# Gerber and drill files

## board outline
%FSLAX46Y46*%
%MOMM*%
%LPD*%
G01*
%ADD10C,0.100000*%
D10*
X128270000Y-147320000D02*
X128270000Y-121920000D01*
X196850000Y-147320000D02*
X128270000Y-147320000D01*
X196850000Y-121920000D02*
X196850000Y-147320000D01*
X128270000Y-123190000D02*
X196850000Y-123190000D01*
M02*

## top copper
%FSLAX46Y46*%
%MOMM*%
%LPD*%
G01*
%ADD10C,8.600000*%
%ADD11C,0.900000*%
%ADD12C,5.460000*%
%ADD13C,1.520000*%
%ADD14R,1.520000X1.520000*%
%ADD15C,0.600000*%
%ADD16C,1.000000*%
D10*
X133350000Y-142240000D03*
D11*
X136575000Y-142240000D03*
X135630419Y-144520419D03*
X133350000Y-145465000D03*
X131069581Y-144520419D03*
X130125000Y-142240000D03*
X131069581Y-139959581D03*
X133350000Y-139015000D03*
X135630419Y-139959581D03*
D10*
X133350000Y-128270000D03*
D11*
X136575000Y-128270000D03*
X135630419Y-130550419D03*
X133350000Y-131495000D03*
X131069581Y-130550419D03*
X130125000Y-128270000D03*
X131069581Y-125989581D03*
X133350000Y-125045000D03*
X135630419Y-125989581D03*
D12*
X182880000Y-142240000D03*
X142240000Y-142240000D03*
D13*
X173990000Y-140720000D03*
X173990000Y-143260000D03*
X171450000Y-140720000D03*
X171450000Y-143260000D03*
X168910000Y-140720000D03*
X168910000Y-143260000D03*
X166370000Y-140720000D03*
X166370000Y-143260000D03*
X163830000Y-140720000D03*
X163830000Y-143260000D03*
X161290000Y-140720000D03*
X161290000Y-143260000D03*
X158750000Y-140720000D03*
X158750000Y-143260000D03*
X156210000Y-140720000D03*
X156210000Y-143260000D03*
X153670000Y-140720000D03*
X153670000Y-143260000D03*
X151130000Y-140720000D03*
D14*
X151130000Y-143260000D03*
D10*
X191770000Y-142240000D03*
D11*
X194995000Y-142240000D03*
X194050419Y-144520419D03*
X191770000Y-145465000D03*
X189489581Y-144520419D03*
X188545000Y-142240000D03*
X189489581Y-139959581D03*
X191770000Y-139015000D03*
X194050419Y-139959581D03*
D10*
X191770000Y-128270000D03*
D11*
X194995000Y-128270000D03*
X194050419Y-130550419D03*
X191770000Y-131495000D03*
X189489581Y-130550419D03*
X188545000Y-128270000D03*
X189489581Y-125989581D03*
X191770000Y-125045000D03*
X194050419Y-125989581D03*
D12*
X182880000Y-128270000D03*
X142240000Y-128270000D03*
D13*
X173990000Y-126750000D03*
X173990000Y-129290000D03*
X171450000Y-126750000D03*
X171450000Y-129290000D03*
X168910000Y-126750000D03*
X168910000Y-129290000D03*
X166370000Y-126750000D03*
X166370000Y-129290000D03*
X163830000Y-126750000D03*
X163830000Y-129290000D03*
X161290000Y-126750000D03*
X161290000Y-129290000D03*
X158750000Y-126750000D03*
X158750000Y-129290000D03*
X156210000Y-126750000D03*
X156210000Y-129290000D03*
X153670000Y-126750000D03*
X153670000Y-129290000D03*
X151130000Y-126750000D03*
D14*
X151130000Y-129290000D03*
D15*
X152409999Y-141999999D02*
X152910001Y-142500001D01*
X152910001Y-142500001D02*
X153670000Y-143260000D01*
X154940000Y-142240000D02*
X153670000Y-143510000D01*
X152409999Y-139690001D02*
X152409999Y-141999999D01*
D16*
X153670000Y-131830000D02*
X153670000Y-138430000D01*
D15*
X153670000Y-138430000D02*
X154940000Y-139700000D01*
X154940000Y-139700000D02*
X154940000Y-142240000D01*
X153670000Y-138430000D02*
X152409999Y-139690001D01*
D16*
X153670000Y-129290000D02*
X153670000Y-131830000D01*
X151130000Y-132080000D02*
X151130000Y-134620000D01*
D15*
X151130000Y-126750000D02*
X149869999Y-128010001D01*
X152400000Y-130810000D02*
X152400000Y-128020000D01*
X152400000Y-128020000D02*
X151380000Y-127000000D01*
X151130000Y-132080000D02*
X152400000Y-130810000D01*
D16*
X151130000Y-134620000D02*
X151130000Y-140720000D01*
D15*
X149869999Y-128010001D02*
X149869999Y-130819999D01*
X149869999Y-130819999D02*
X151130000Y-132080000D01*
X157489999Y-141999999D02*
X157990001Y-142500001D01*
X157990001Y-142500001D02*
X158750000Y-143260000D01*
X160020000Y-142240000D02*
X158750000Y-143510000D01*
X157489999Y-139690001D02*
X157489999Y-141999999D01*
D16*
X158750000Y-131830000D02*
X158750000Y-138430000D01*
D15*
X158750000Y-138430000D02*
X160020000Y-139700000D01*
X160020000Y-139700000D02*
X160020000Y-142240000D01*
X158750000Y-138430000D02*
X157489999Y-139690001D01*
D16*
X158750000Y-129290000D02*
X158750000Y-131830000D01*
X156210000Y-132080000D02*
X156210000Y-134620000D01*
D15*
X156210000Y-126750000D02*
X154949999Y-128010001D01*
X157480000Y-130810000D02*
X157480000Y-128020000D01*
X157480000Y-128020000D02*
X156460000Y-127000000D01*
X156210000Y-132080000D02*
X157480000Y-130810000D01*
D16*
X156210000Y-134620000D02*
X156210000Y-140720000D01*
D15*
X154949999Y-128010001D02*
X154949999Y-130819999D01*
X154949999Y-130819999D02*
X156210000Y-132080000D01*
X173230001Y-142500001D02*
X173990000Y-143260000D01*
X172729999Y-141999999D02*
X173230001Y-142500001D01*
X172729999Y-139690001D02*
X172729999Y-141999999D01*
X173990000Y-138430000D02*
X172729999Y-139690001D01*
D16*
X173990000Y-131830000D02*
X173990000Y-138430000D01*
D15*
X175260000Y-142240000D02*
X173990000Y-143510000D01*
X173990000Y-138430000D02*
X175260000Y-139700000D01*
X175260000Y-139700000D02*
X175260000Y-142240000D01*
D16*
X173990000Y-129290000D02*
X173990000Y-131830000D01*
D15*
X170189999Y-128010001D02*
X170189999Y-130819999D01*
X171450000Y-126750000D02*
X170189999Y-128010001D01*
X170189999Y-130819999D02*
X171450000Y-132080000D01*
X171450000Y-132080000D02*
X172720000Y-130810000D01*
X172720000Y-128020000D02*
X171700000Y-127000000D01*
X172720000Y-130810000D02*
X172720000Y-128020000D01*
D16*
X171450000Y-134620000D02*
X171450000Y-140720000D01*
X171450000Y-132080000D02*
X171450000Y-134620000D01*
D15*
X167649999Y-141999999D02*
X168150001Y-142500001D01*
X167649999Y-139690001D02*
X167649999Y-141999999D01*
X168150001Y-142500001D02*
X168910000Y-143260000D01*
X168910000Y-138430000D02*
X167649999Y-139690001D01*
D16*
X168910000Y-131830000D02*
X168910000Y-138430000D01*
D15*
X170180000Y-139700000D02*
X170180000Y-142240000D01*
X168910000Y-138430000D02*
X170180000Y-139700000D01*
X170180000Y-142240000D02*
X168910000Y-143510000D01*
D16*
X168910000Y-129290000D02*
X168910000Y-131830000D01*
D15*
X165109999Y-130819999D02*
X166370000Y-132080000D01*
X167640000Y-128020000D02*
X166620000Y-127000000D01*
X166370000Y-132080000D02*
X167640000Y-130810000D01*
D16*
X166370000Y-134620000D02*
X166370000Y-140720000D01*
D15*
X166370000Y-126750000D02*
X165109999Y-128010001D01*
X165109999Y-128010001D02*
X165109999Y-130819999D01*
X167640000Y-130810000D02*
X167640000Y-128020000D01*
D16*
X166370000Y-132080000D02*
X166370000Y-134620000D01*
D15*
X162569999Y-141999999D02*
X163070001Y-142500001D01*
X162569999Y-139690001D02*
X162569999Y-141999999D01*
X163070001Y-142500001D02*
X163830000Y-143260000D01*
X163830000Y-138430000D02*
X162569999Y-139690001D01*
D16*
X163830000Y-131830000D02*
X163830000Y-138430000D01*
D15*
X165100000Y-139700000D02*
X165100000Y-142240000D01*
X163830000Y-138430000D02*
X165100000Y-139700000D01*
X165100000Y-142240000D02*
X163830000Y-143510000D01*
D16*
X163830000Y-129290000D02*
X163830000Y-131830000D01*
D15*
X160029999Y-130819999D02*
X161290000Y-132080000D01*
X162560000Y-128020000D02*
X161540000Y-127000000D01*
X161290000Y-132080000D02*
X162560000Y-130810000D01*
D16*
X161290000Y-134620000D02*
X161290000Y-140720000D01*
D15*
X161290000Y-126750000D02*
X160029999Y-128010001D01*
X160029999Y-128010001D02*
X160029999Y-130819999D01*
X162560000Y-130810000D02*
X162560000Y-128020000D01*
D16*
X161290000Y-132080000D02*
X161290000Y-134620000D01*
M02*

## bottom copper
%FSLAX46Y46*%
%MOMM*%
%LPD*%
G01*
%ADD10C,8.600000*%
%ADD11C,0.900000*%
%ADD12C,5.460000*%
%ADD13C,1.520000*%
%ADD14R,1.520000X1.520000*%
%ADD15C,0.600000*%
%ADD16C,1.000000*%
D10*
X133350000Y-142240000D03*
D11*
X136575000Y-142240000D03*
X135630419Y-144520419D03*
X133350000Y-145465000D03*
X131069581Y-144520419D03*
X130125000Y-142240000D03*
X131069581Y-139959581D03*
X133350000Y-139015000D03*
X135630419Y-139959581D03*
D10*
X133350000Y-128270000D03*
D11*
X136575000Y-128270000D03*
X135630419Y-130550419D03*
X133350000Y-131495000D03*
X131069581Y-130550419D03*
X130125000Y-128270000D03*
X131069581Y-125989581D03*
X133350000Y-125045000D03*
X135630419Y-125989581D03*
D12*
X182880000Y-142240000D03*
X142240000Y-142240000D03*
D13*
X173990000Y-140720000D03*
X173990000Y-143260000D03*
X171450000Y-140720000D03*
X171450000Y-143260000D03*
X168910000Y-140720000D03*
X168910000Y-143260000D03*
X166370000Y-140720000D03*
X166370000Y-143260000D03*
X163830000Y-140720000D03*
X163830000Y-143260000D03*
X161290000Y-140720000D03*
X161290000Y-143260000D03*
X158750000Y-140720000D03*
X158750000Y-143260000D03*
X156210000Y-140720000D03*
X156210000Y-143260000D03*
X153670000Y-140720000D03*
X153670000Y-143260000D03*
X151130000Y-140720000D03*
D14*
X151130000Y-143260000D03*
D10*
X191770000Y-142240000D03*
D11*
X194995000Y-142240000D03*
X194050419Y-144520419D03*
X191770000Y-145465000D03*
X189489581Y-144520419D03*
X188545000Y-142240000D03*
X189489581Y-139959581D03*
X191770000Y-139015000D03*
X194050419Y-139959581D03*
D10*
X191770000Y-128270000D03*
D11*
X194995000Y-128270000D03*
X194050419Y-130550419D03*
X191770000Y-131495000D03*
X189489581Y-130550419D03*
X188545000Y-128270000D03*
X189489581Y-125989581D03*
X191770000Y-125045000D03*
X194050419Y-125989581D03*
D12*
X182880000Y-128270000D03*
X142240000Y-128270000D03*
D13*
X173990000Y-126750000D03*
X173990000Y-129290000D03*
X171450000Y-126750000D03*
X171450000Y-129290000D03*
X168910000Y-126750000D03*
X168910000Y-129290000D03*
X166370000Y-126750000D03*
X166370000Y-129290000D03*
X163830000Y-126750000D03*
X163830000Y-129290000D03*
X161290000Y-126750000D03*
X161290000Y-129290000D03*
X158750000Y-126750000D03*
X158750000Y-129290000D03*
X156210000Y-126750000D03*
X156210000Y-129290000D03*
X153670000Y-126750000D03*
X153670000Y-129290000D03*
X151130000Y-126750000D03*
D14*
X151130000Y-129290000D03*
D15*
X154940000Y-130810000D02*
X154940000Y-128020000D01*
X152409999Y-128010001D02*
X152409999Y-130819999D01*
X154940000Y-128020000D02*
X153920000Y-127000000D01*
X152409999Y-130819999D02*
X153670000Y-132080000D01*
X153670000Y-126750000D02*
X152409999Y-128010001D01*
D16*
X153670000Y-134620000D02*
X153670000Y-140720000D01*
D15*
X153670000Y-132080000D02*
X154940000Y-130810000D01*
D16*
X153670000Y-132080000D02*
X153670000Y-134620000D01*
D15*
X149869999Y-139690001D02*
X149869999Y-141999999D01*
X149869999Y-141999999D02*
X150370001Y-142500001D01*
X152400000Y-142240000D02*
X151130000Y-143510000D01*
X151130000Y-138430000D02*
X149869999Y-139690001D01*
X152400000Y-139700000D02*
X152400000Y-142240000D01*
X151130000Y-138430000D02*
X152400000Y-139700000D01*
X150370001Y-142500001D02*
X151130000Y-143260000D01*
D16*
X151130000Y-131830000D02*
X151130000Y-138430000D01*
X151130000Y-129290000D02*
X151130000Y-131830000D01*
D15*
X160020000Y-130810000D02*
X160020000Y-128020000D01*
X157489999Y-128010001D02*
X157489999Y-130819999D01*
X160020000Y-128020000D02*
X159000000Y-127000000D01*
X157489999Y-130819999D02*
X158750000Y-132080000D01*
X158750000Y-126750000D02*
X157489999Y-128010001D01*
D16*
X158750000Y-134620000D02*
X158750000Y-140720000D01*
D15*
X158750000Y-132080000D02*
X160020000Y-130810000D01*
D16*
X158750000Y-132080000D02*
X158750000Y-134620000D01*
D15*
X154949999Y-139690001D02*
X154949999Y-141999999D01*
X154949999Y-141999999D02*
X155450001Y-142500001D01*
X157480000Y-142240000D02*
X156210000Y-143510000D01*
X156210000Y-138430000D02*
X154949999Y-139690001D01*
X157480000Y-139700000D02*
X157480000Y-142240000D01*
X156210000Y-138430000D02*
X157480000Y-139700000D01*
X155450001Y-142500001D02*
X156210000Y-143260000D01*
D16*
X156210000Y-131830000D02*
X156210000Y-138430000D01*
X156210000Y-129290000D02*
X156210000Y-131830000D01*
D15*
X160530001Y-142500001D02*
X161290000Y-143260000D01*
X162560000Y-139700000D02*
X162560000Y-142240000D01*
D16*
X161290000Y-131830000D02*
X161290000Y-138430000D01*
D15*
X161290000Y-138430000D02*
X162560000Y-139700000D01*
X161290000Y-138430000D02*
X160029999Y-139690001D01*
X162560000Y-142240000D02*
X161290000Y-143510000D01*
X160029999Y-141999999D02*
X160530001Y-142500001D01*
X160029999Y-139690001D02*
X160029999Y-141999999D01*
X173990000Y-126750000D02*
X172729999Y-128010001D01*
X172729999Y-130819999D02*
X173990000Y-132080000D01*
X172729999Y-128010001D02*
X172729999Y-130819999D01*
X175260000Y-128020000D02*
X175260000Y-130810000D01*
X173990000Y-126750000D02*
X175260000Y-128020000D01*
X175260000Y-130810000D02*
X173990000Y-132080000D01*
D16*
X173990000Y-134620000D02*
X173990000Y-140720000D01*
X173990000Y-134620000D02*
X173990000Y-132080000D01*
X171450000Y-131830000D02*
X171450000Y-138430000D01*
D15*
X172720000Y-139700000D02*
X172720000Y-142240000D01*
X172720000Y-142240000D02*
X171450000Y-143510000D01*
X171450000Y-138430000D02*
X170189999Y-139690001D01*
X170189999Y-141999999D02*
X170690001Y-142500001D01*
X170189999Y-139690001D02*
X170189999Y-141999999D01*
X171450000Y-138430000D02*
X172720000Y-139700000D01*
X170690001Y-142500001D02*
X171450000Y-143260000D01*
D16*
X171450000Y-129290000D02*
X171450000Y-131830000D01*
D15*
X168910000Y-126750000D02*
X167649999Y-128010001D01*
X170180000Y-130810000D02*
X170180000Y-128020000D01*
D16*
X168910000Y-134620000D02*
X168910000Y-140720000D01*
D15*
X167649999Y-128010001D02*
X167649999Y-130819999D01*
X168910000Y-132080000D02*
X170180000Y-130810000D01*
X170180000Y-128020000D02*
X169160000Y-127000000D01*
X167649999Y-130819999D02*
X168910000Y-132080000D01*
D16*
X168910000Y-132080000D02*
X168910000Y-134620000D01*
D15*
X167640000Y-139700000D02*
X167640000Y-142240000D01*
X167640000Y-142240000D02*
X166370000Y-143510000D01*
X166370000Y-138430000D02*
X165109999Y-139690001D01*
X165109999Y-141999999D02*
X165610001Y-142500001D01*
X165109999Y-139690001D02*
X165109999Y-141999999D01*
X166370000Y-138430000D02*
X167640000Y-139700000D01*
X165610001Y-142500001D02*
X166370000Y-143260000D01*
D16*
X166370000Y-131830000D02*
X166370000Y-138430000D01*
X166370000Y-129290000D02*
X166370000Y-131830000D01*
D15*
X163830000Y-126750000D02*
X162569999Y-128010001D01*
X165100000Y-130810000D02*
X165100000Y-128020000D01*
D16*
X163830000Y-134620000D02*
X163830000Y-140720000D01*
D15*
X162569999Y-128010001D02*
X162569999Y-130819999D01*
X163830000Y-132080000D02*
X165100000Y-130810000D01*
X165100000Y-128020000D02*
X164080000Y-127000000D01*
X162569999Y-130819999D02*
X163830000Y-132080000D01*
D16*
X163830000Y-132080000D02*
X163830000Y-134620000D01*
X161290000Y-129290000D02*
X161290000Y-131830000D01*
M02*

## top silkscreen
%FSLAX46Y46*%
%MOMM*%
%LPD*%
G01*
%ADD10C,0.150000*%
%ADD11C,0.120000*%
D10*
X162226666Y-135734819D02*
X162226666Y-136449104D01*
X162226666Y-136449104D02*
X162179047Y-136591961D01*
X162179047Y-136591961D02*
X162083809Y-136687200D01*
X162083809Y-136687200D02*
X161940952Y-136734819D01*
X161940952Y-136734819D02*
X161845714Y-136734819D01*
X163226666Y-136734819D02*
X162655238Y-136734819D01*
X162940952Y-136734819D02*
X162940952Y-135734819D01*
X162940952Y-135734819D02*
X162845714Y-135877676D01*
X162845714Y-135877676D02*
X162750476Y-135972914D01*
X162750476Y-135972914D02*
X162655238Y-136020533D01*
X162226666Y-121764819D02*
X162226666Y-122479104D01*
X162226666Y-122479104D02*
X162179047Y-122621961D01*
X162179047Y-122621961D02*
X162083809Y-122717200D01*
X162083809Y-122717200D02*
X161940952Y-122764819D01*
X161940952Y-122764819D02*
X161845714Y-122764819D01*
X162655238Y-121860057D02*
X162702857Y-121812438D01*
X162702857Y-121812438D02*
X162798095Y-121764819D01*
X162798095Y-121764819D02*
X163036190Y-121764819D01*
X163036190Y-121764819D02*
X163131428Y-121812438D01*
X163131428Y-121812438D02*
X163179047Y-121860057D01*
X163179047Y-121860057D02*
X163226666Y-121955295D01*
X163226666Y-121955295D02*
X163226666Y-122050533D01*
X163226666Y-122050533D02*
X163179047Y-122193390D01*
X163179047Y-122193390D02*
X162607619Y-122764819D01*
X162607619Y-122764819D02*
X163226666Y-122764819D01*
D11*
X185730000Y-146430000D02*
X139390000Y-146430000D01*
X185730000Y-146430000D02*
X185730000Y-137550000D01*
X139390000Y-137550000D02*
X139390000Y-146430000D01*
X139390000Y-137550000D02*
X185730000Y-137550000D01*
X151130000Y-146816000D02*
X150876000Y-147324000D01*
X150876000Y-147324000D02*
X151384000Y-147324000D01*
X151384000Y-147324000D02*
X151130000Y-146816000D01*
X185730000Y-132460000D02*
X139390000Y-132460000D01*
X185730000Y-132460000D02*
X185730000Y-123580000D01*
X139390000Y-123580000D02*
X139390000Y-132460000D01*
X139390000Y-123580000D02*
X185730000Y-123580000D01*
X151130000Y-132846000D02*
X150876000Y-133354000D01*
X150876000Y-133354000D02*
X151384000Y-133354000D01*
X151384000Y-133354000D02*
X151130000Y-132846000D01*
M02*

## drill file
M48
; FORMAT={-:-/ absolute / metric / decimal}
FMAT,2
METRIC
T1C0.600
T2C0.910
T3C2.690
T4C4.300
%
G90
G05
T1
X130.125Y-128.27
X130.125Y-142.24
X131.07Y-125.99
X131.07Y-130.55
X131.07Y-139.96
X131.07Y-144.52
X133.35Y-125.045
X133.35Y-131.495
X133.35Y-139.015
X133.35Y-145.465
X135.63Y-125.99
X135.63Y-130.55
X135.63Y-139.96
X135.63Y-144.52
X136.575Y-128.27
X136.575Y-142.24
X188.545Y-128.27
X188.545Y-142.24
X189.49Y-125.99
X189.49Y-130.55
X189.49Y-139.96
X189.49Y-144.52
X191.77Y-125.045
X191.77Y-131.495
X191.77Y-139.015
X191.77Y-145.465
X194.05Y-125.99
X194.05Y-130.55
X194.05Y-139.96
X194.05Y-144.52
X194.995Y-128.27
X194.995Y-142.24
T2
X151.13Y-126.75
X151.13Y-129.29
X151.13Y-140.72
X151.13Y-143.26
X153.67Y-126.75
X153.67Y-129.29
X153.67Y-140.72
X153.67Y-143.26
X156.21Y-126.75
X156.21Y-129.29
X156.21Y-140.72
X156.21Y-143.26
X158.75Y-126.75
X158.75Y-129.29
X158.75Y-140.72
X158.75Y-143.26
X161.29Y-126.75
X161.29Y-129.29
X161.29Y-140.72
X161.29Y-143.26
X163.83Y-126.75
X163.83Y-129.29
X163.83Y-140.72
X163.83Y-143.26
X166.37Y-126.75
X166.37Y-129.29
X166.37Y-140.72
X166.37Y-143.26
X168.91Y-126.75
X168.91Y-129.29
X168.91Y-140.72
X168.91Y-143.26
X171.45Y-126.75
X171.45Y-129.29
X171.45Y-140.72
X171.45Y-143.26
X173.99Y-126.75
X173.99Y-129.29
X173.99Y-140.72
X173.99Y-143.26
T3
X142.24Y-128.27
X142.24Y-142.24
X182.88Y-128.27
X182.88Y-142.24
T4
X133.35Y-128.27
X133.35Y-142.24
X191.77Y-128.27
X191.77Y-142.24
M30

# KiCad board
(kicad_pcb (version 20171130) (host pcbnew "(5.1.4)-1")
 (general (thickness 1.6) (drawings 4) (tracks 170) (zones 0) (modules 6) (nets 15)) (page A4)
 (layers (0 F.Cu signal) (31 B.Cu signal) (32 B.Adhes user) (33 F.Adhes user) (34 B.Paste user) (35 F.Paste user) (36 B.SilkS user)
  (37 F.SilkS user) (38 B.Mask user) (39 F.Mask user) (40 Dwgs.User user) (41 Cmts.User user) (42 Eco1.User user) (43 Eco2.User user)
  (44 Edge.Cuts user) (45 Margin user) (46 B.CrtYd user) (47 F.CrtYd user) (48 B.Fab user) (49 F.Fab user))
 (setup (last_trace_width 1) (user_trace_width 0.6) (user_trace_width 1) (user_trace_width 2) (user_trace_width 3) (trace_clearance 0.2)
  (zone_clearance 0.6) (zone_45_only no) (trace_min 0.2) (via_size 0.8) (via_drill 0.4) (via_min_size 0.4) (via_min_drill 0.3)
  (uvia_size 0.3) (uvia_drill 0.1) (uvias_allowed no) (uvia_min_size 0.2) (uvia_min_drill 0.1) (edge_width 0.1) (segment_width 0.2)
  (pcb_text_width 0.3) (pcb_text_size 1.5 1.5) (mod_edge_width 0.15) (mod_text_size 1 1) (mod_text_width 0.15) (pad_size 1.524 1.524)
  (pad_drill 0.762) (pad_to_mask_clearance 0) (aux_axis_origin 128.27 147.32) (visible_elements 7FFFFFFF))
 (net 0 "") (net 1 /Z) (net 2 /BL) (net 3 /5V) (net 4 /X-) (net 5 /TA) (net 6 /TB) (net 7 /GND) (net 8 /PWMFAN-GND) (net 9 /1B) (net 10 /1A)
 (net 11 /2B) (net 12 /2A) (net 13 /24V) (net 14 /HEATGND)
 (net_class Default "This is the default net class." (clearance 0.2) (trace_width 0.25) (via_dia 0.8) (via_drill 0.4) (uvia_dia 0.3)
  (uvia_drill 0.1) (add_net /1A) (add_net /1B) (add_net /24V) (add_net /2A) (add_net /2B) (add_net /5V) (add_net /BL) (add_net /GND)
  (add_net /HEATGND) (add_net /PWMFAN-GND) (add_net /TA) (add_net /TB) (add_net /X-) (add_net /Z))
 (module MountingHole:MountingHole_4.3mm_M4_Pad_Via (layer F.Cu) (at 133.35 142.24)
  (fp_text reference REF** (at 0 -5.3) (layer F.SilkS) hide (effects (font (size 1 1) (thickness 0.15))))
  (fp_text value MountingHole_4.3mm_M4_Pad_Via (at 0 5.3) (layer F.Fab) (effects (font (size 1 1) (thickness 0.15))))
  (pad 1 thru_hole circle (at 0 0) (size 8.6 8.6) (drill 4.3) (layers *.Cu *.Mask))
  (pad 1 thru_hole circle (at 3.225 0) (size 0.9 0.9) (drill 0.6) (layers *.Cu *.Mask))
  (pad 1 thru_hole circle (at 2.280419 2.280419) (size 0.9 0.9) (drill 0.6) (layers *.Cu *.Mask))
  (pad 1 thru_hole circle (at 0 3.225) (size 0.9 0.9) (drill 0.6) (layers *.Cu *.Mask))
  (pad 1 thru_hole circle (at -2.280419 2.280419) (size 0.9 0.9) (drill 0.6) (layers *.Cu *.Mask))
  (pad 1 thru_hole circle (at -3.225 0) (size 0.9 0.9) (drill 0.6) (layers *.Cu *.Mask))
  (pad 1 thru_hole circle (at -2.280419 -2.280419) (size 0.9 0.9) (drill 0.6) (layers *.Cu *.Mask))
  (pad 1 thru_hole circle (at 0 -3.225) (size 0.9 0.9) (drill 0.6) (layers *.Cu *.Mask))
  (pad 1 thru_hole circle (at 2.280419 -2.280419) (size 0.9 0.9) (drill 0.6) (layers *.Cu *.Mask)))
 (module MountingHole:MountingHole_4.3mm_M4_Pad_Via (layer F.Cu) (at 133.35 128.27)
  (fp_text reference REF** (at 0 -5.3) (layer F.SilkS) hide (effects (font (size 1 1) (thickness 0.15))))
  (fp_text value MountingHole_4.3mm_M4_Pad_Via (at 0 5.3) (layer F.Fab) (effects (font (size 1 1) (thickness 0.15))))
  (pad 1 thru_hole circle (at 0 0) (size 8.6 8.6) (drill 4.3) (layers *.Cu *.Mask))
  (pad 1 thru_hole circle (at 3.225 0) (size 0.9 0.9) (drill 0.6) (layers *.Cu *.Mask))
  (pad 1 thru_hole circle (at 2.280419 2.280419) (size 0.9 0.9) (drill 0.6) (layers *.Cu *.Mask))
  (pad 1 thru_hole circle (at 0 3.225) (size 0.9 0.9) (drill 0.6) (layers *.Cu *.Mask))
  (pad 1 thru_hole circle (at -2.280419 2.280419) (size 0.9 0.9) (drill 0.6) (layers *.Cu *.Mask))
  (pad 1 thru_hole circle (at -3.225 0) (size 0.9 0.9) (drill 0.6) (layers *.Cu *.Mask))
  (pad 1 thru_hole circle (at -2.280419 -2.280419) (size 0.9 0.9) (drill 0.6) (layers *.Cu *.Mask))
  (pad 1 thru_hole circle (at 0 -3.225) (size 0.9 0.9) (drill 0.6) (layers *.Cu *.Mask))
  (pad 1 thru_hole circle (at 2.280419 -2.280419) (size 0.9 0.9) (drill 0.6) (layers *.Cu *.Mask)))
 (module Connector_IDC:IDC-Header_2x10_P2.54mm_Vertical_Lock (layer F.Cu) (at 151.13 143.26 90)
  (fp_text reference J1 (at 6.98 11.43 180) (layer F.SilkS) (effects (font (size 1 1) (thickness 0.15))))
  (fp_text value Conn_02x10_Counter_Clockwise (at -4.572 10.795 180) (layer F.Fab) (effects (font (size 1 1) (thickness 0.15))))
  (fp_line (start -3.17 34.6) (end -3.17 -11.74) (layer F.SilkS) (width 0.12))
  (fp_line (start -3.17 34.6) (end 5.71 34.6) (layer F.SilkS) (width 0.12))
  (fp_line (start 5.71 -11.74) (end -3.17 -11.74) (layer F.SilkS) (width 0.12))
  (fp_line (start 5.71 -11.74) (end 5.71 34.6) (layer F.SilkS) (width 0.12))
  (fp_line (start -3.556 0) (end -4.064 -0.254) (layer F.SilkS) (width 0.12))
  (fp_line (start -4.064 -0.254) (end -4.064 0.254) (layer F.SilkS) (width 0.12))
  (fp_line (start -4.064 0.254) (end -3.556 0) (layer F.SilkS) (width 0.12))
  (pad "" thru_hole circle (at 1.02 31.75) (size 5.46 5.46) (drill 2.69) (layers *.Cu *.Mask))
  (pad "" thru_hole circle (at 1.02 -8.89) (size 5.46 5.46) (drill 2.69) (layers *.Cu *.Mask))
  (pad 20 thru_hole circle (at 2.54 22.86) (size 1.52 1.52) (drill 0.91) (layers *.Cu *.Mask) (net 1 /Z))
  (pad 19 thru_hole circle (at 0 22.86) (size 1.52 1.52) (drill 0.91) (layers *.Cu *.Mask) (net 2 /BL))
  (pad 18 thru_hole circle (at 2.54 20.32) (size 1.52 1.52) (drill 0.91) (layers *.Cu *.Mask) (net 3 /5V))
  (pad 17 thru_hole circle (at 0 20.32) (size 1.52 1.52) (drill 0.91) (layers *.Cu *.Mask) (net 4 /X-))
  (pad 16 thru_hole circle (at 2.54 17.78) (size 1.52 1.52) (drill 0.91) (layers *.Cu *.Mask) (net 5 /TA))
  (pad 15 thru_hole circle (at 0 17.78) (size 1.52 1.52) (drill 0.91) (layers *.Cu *.Mask) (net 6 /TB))
  (pad 14 thru_hole circle (at 2.54 15.24) (size 1.52 1.52) (drill 0.91) (layers *.Cu *.Mask) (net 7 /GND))
  (pad 13 thru_hole circle (at 0 15.24) (size 1.52 1.52) (drill 0.91) (layers *.Cu *.Mask) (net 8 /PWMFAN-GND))
  (pad 12 thru_hole circle (at 2.54 12.7) (size 1.52 1.52) (drill 0.91) (layers *.Cu *.Mask) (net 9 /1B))
  (pad 11 thru_hole circle (at 0 12.7) (size 1.52 1.52) (drill 0.91) (layers *.Cu *.Mask) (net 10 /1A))
  (pad 10 thru_hole circle (at 2.54 10.16) (size 1.52 1.52) (drill 0.91) (layers *.Cu *.Mask) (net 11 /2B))
  (pad 9 thru_hole circle (at 0 10.16) (size 1.52 1.52) (drill 0.91) (layers *.Cu *.Mask) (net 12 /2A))
  (pad 8 thru_hole circle (at 2.54 7.62) (size 1.52 1.52) (drill 0.91) (layers *.Cu *.Mask) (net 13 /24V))
  (pad 7 thru_hole circle (at 0 7.62) (size 1.52 1.52) (drill 0.91) (layers *.Cu *.Mask) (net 13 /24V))
  (pad 6 thru_hole circle (at 2.54 5.08) (size 1.52 1.52) (drill 0.91) (layers *.Cu *.Mask) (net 13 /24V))
  (pad 5 thru_hole circle (at 0 5.08) (size 1.52 1.52) (drill 0.91) (layers *.Cu *.Mask) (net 13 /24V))
  (pad 4 thru_hole circle (at 2.54 2.54) (size 1.52 1.52) (drill 0.91) (layers *.Cu *.Mask) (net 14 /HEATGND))
  (pad 3 thru_hole circle (at 0 2.54) (size 1.52 1.52) (drill 0.91) (layers *.Cu *.Mask) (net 14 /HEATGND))
  (pad 2 thru_hole circle (at 2.54 0) (size 1.52 1.52) (drill 0.91) (layers *.Cu *.Mask) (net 14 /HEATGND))
  (pad 1 thru_hole rect (at 0 0) (size 1.52 1.52) (drill 0.91) (layers *.Cu *.Mask) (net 14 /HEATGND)))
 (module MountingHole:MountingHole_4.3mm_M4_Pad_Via (layer F.Cu) (at 191.77 142.24)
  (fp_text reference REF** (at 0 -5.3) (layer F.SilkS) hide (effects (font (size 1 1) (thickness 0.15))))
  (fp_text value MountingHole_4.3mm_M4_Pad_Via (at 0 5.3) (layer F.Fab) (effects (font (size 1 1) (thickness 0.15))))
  (pad 1 thru_hole circle (at 0 0) (size 8.6 8.6) (drill 4.3) (layers *.Cu *.Mask))
  (pad 1 thru_hole circle (at 3.225 0) (size 0.9 0.9) (drill 0.6) (layers *.Cu *.Mask))
  (pad 1 thru_hole circle (at 2.280419 2.280419) (size 0.9 0.9) (drill 0.6) (layers *.Cu *.Mask))
  (pad 1 thru_hole circle (at 0 3.225) (size 0.9 0.9) (drill 0.6) (layers *.Cu *.Mask))
  (pad 1 thru_hole circle (at -2.280419 2.280419) (size 0.9 0.9) (drill 0.6) (layers *.Cu *.Mask))
  (pad 1 thru_hole circle (at -3.225 0) (size 0.9 0.9) (drill 0.6) (layers *.Cu *.Mask))
  (pad 1 thru_hole circle (at -2.280419 -2.280419) (size 0.9 0.9) (drill 0.6) (layers *.Cu *.Mask))
  (pad 1 thru_hole circle (at 0 -3.225) (size 0.9 0.9) (drill 0.6) (layers *.Cu *.Mask))
  (pad 1 thru_hole circle (at 2.280419 -2.280419) (size 0.9 0.9) (drill 0.6) (layers *.Cu *.Mask)))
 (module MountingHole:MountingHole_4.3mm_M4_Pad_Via (layer F.Cu) (at 191.77 128.27)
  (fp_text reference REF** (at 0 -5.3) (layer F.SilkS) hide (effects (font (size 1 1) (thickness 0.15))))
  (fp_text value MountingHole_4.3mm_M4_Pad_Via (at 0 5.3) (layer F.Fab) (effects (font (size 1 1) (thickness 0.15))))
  (pad 1 thru_hole circle (at 0 0) (size 8.6 8.6) (drill 4.3) (layers *.Cu *.Mask))
  (pad 1 thru_hole circle (at 3.225 0) (size 0.9 0.9) (drill 0.6) (layers *.Cu *.Mask))
  (pad 1 thru_hole circle (at 2.280419 2.280419) (size 0.9 0.9) (drill 0.6) (layers *.Cu *.Mask))
  (pad 1 thru_hole circle (at 0 3.225) (size 0.9 0.9) (drill 0.6) (layers *.Cu *.Mask))
  (pad 1 thru_hole circle (at -2.280419 2.280419) (size 0.9 0.9) (drill 0.6) (layers *.Cu *.Mask))
  (pad 1 thru_hole circle (at -3.225 0) (size 0.9 0.9) (drill 0.6) (layers *.Cu *.Mask))
  (pad 1 thru_hole circle (at -2.280419 -2.280419) (size 0.9 0.9) (drill 0.6) (layers *.Cu *.Mask))
  (pad 1 thru_hole circle (at 0 -3.225) (size 0.9 0.9) (drill 0.6) (layers *.Cu *.Mask))
  (pad 1 thru_hole circle (at 2.280419 -2.280419) (size 0.9 0.9) (drill 0.6) (layers *.Cu *.Mask)))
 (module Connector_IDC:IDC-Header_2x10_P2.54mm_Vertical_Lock (layer F.Cu) (at 151.13 129.29 90)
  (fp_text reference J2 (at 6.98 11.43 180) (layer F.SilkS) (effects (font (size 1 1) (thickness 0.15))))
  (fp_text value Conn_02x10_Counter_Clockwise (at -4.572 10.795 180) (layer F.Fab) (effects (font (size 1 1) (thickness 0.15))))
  (fp_line (start -3.17 34.6) (end -3.17 -11.74) (layer F.SilkS) (width 0.12))
  (fp_line (start -3.17 34.6) (end 5.71 34.6) (layer F.SilkS) (width 0.12))
  (fp_line (start 5.71 -11.74) (end -3.17 -11.74) (layer F.SilkS) (width 0.12))
  (fp_line (start 5.71 -11.74) (end 5.71 34.6) (layer F.SilkS) (width 0.12))
  (fp_line (start -3.556 0) (end -4.064 -0.254) (layer F.SilkS) (width 0.12))
  (fp_line (start -4.064 -0.254) (end -4.064 0.254) (layer F.SilkS) (width 0.12))
  (fp_line (start -4.064 0.254) (end -3.556 0) (layer F.SilkS) (width 0.12))
  (pad "" thru_hole circle (at 1.02 31.75) (size 5.46 5.46) (drill 2.69) (layers *.Cu *.Mask))
  (pad "" thru_hole circle (at 1.02 -8.89) (size 5.46 5.46) (drill 2.69) (layers *.Cu *.Mask))
  (pad 20 thru_hole circle (at 2.54 22.86) (size 1.52 1.52) (drill 0.91) (layers *.Cu *.Mask) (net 1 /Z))
  (pad 19 thru_hole circle (at 0 22.86) (size 1.52 1.52) (drill 0.91) (layers *.Cu *.Mask) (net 2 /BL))
  (pad 18 thru_hole circle (at 2.54 20.32) (size 1.52 1.52) (drill 0.91) (layers *.Cu *.Mask) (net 3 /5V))
  (pad 17 thru_hole circle (at 0 20.32) (size 1.52 1.52) (drill 0.91) (layers *.Cu *.Mask) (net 4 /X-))
  (pad 16 thru_hole circle (at 2.54 17.78) (size 1.52 1.52) (drill 0.91) (layers *.Cu *.Mask) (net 5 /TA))
  (pad 15 thru_hole circle (at 0 17.78) (size 1.52 1.52) (drill 0.91) (layers *.Cu *.Mask) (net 6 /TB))
  (pad 14 thru_hole circle (at 2.54 15.24) (size 1.52 1.52) (drill 0.91) (layers *.Cu *.Mask) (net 7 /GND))
  (pad 13 thru_hole circle (at 0 15.24) (size 1.52 1.52) (drill 0.91) (layers *.Cu *.Mask) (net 8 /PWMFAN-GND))
  (pad 12 thru_hole circle (at 2.54 12.7) (size 1.52 1.52) (drill 0.91) (layers *.Cu *.Mask) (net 9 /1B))
  (pad 11 thru_hole circle (at 0 12.7) (size 1.52 1.52) (drill 0.91) (layers *.Cu *.Mask) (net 10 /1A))
  (pad 10 thru_hole circle (at 2.54 10.16) (size 1.52 1.52) (drill 0.91) (layers *.Cu *.Mask) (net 11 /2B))
  (pad 9 thru_hole circle (at 0 10.16) (size 1.52 1.52) (drill 0.91) (layers *.Cu *.Mask) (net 12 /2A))
  (pad 8 thru_hole circle (at 2.54 7.62) (size 1.52 1.52) (drill 0.91) (layers *.Cu *.Mask) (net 13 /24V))
  (pad 7 thru_hole circle (at 0 7.62) (size 1.52 1.52) (drill 0.91) (layers *.Cu *.Mask) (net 13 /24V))
  (pad 6 thru_hole circle (at 2.54 5.08) (size 1.52 1.52) (drill 0.91) (layers *.Cu *.Mask) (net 13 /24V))
  (pad 5 thru_hole circle (at 0 5.08) (size 1.52 1.52) (drill 0.91) (layers *.Cu *.Mask) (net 13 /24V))
  (pad 4 thru_hole circle (at 2.54 2.54) (size 1.52 1.52) (drill 0.91) (layers *.Cu *.Mask) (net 14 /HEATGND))
  (pad 3 thru_hole circle (at 0 2.54) (size 1.52 1.52) (drill 0.91) (layers *.Cu *.Mask) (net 14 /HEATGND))
  (pad 2 thru_hole circle (at 2.54 0) (size 1.52 1.52) (drill 0.91) (layers *.Cu *.Mask) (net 14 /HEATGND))
  (pad 1 thru_hole rect (at 0 0) (size 1.52 1.52) (drill 0.91) (layers *.Cu *.Mask) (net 14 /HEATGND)))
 (gr_line (start 128.27 147.32) (end 128.27 121.92) (layer Edge.Cuts) (width 0.1))
 (gr_line (start 196.85 147.32) (end 128.27 147.32) (layer Edge.Cuts) (width 0.1))
 (gr_line (start 196.85 121.92) (end 196.85 147.32) (layer Edge.Cuts) (width 0.1))
 (gr_line (start 128.27 123.19) (end 196.85 123.19) (layer Edge.Cuts) (width 0.1))
 (segment (start 154.94 130.81) (end 154.94 128.02) (width 0.6) (layer B.Cu) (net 14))
 (segment (start 152.409999 128.010001) (end 152.409999 130.819999) (width 0.6) (layer B.Cu) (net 14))
 (segment (start 154.94 128.02) (end 153.92 127) (width 0.6) (layer B.Cu) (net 14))
 (segment (start 152.409999 130.819999) (end 153.67 132.08) (width 0.6) (layer B.Cu) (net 14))
 (segment (start 153.67 126.75) (end 152.409999 128.010001) (width 0.6) (layer B.Cu) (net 14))
 (segment (start 153.67 134.62) (end 153.67 140.72) (width 1) (layer B.Cu) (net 14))
 (segment (start 153.67 132.08) (end 154.94 130.81) (width 0.6) (layer B.Cu) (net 14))
 (segment (start 153.67 132.08) (end 153.67 134.62) (width 1) (layer B.Cu) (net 14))
 (segment (start 149.869999 139.690001) (end 149.869999 141.999999) (width 0.6) (layer B.Cu) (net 14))
 (segment (start 149.869999 141.999999) (end 150.370001 142.500001) (width 0.6) (layer B.Cu) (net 14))
 (segment (start 152.4 142.24) (end 151.13 143.51) (width 0.6) (layer B.Cu) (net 14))
 (segment (start 151.13 138.43) (end 149.869999 139.690001) (width 0.6) (layer B.Cu) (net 14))
 (segment (start 152.4 139.7) (end 152.4 142.24) (width 0.6) (layer B.Cu) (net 14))
 (segment (start 151.13 138.43) (end 152.4 139.7) (width 0.6) (layer B.Cu) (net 14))
 (segment (start 150.370001 142.500001) (end 151.13 143.26) (width 0.6) (layer B.Cu) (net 14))
 (segment (start 151.13 131.83) (end 151.13 138.43) (width 1) (layer B.Cu) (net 14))
 (segment (start 151.13 129.29) (end 151.13 131.83) (width 1) (layer B.Cu) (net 14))
 (segment (start 160.02 130.81) (end 160.02 128.02) (width 0.6) (layer B.Cu) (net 13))
 (segment (start 157.489999 128.010001) (end 157.489999 130.819999) (width 0.6) (layer B.Cu) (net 13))
 (segment (start 160.02 128.02) (end 159 127) (width 0.6) (layer B.Cu) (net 13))
 (segment (start 157.489999 130.819999) (end 158.75 132.08) (width 0.6) (layer B.Cu) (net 13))
 (segment (start 158.75 126.75) (end 157.489999 128.010001) (width 0.6) (layer B.Cu) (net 13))
 (segment (start 158.75 134.62) (end 158.75 140.72) (width 1) (layer B.Cu) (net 13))
 (segment (start 158.75 132.08) (end 160.02 130.81) (width 0.6) (layer B.Cu) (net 13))
 (segment (start 158.75 132.08) (end 158.75 134.62) (width 1) (layer B.Cu) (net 13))
 (segment (start 154.949999 139.690001) (end 154.949999 141.999999) (width 0.6) (layer B.Cu) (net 13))
 (segment (start 154.949999 141.999999) (end 155.450001 142.500001) (width 0.6) (layer B.Cu) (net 13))
 (segment (start 157.48 142.24) (end 156.21 143.51) (width 0.6) (layer B.Cu) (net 13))
 (segment (start 156.21 138.43) (end 154.949999 139.690001) (width 0.6) (layer B.Cu) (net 13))
 (segment (start 157.48 139.7) (end 157.48 142.24) (width 0.6) (layer B.Cu) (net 13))
 (segment (start 156.21 138.43) (end 157.48 139.7) (width 0.6) (layer B.Cu) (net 13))
 (segment (start 155.450001 142.500001) (end 156.21 143.26) (width 0.6) (layer B.Cu) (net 13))
 (segment (start 156.21 131.83) (end 156.21 138.43) (width 1) (layer B.Cu) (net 13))
 (segment (start 156.21 129.29) (end 156.21 131.83) (width 1) (layer B.Cu) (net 13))
 (segment (start 152.409999 141.999999) (end 152.910001 142.500001) (width 0.6) (layer F.Cu) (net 14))
 (segment (start 152.910001 142.500001) (end 153.67 143.26) (width 0.6) (layer F.Cu) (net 14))
 (segment (start 154.94 142.24) (end 153.67 143.51) (width 0.6) (layer F.Cu) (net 14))
 (segment (start 152.409999 139.690001) (end 152.409999 141.999999) (width 0.6) (layer F.Cu) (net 14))
 (segment (start 153.67 131.83) (end 153.67 138.43) (width 1) (layer F.Cu) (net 14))
 (segment (start 153.67 138.43) (end 154.94 139.7) (width 0.6) (layer F.Cu) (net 14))
 (segment (start 154.94 139.7) (end 154.94 142.24) (width 0.6) (layer F.Cu) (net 14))
 (segment (start 153.67 138.43) (end 152.409999 139.690001) (width 0.6) (layer F.Cu) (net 14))
 (segment (start 153.67 129.29) (end 153.67 131.83) (width 1) (layer F.Cu) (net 14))
 (segment (start 151.13 132.08) (end 151.13 134.62) (width 1) (layer F.Cu) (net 14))
 (segment (start 151.13 126.75) (end 149.869999 128.010001) (width 0.6) (layer F.Cu) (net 14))
 (segment (start 152.4 130.81) (end 152.4 128.02) (width 0.6) (layer F.Cu) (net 14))
 (segment (start 152.4 128.02) (end 151.38 127) (width 0.6) (layer F.Cu) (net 14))
 (segment (start 151.13 132.08) (end 152.4 130.81) (width 0.6) (layer F.Cu) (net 14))
 (segment (start 151.13 134.62) (end 151.13 140.72) (width 1) (layer F.Cu) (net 14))
 (segment (start 149.869999 128.010001) (end 149.869999 130.819999) (width 0.6) (layer F.Cu) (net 14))
 (segment (start 149.869999 130.819999) (end 151.13 132.08) (width 0.6) (layer F.Cu) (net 14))
 (segment (start 157.489999 141.999999) (end 157.990001 142.500001) (width 0.6) (layer F.Cu) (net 13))
 (segment (start 157.990001 142.500001) (end 158.75 143.26) (width 0.6) (layer F.Cu) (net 13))
 (segment (start 160.02 142.24) (end 158.75 143.51) (width 0.6) (layer F.Cu) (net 13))
 (segment (start 157.489999 139.690001) (end 157.489999 141.999999) (width 0.6) (layer F.Cu) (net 13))
 (segment (start 158.75 131.83) (end 158.75 138.43) (width 1) (layer F.Cu) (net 13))
 (segment (start 158.75 138.43) (end 160.02 139.7) (width 0.6) (layer F.Cu) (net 13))
 (segment (start 160.02 139.7) (end 160.02 142.24) (width 0.6) (layer F.Cu) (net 13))
 (segment (start 158.75 138.43) (end 157.489999 139.690001) (width 0.6) (layer F.Cu) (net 13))
 (segment (start 158.75 129.29) (end 158.75 131.83) (width 1) (layer F.Cu) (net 13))
 (segment (start 156.21 132.08) (end 156.21 134.62) (width 1) (layer F.Cu) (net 13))
 (segment (start 156.21 126.75) (end 154.949999 128.010001) (width 0.6) (layer F.Cu) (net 13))
 (segment (start 157.48 130.81) (end 157.48 128.02) (width 0.6) (layer F.Cu) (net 13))
 (segment (start 157.48 128.02) (end 156.46 127) (width 0.6) (layer F.Cu) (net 13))
 (segment (start 156.21 132.08) (end 157.48 130.81) (width 0.6) (layer F.Cu) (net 13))
 (segment (start 156.21 134.62) (end 156.21 140.72) (width 1) (layer F.Cu) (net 13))
 (segment (start 154.949999 128.010001) (end 154.949999 130.819999) (width 0.6) (layer F.Cu) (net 13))
 (segment (start 154.949999 130.819999) (end 156.21 132.08) (width 0.6) (layer F.Cu) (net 13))
 (segment (start 160.530001 142.500001) (end 161.29 143.26) (width 0.6) (layer B.Cu) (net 12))
 (segment (start 162.56 139.7) (end 162.56 142.24) (width 0.6) (layer B.Cu) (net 12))
 (segment (start 161.29 131.83) (end 161.29 138.43) (width 1) (layer B.Cu) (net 12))
 (segment (start 161.29 138.43) (end 162.56 139.7) (width 0.6) (layer B.Cu) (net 12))
 (segment (start 161.29 138.43) (end 160.029999 139.690001) (width 0.6) (layer B.Cu) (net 12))
 (segment (start 162.56 142.24) (end 161.29 143.51) (width 0.6) (layer B.Cu) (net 12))
 (segment (start 160.029999 141.999999) (end 160.530001 142.500001) (width 0.6) (layer B.Cu) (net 12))
 (segment (start 160.029999 139.690001) (end 160.029999 141.999999) (width 0.6) (layer B.Cu) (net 12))
 (segment (start 173.99 126.75) (end 172.729999 128.010001) (width 0.6) (layer B.Cu) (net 1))
 (segment (start 172.729999 130.819999) (end 173.99 132.08) (width 0.6) (layer B.Cu) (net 1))
 (segment (start 172.729999 128.010001) (end 172.729999 130.819999) (width 0.6) (layer B.Cu) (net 1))
 (segment (start 175.26 128.02) (end 175.26 130.81) (width 0.6) (layer B.Cu) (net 1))
 (segment (start 173.99 126.75) (end 175.26 128.02) (width 0.6) (layer B.Cu) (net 1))
 (segment (start 175.26 130.81) (end 173.99 132.08) (width 0.6) (layer B.Cu) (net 1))
 (segment (start 173.99 134.62) (end 173.99 140.72) (width 1) (layer B.Cu) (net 1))
 (segment (start 173.99 134.62) (end 173.99 132.08) (width 1) (layer B.Cu) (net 1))
 (segment (start 173.230001 142.500001) (end 173.99 143.26) (width 0.6) (layer F.Cu) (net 2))
 (segment (start 172.729999 141.999999) (end 173.230001 142.500001) (width 0.6) (layer F.Cu) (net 2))
 (segment (start 172.729999 139.690001) (end 172.729999 141.999999) (width 0.6) (layer F.Cu) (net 2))
 (segment (start 173.99 138.43) (end 172.729999 139.690001) (width 0.6) (layer F.Cu) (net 2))
 (segment (start 173.99 131.83) (end 173.99 138.43) (width 1) (layer F.Cu) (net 2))
 (segment (start 175.26 142.24) (end 173.99 143.51) (width 0.6) (layer F.Cu) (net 2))
 (segment (start 173.99 138.43) (end 175.26 139.7) (width 0.6) (layer F.Cu) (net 2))
 (segment (start 175.26 139.7) (end 175.26 142.24) (width 0.6) (layer F.Cu) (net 2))
 (segment (start 173.99 129.29) (end 173.99 131.83) (width 1) (layer F.Cu) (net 2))
 (segment (start 170.189999 128.010001) (end 170.189999 130.819999) (width 0.6) (layer F.Cu) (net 3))
 (segment (start 171.45 126.75) (end 170.189999 128.010001) (width 0.6) (layer F.Cu) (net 3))
 (segment (start 170.189999 130.819999) (end 171.45 132.08) (width 0.6) (layer F.Cu) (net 3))
 (segment (start 171.45 132.08) (end 172.72 130.81) (width 0.6) (layer F.Cu) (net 3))
 (segment (start 172.72 128.02) (end 171.7 127) (width 0.6) (layer F.Cu) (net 3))
 (segment (start 172.72 130.81) (end 172.72 128.02) (width 0.6) (layer F.Cu) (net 3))
 (segment (start 171.45 134.62) (end 171.45 140.72) (width 1) (layer F.Cu) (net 3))
 (segment (start 171.45 132.08) (end 171.45 134.62) (width 1) (layer F.Cu) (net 3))
 (segment (start 171.45 131.83) (end 171.45 138.43) (width 1) (layer B.Cu) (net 4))
 (segment (start 172.72 139.7) (end 172.72 142.24) (width 0.6) (layer B.Cu) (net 4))
 (segment (start 172.72 142.24) (end 171.45 143.51) (width 0.6) (layer B.Cu) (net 4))
 (segment (start 171.45 138.43) (end 170.189999 139.690001) (width 0.6) (layer B.Cu) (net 4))
 (segment (start 170.189999 141.999999) (end 170.690001 142.500001) (width 0.6) (layer B.Cu) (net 4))
 (segment (start 170.189999 139.690001) (end 170.189999 141.999999) (width 0.6) (layer B.Cu) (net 4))
 (segment (start 171.45 138.43) (end 172.72 139.7) (width 0.6) (layer B.Cu) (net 4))
 (segment (start 170.690001 142.500001) (end 171.45 143.26) (width 0.6) (layer B.Cu) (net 4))
 (segment (start 171.45 129.29) (end 171.45 131.83) (width 1) (layer B.Cu) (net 4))
 (segment (start 168.91 126.75) (end 167.649999 128.010001) (width 0.6) (layer B.Cu) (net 5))
 (segment (start 170.18 130.81) (end 170.18 128.02) (width 0.6) (layer B.Cu) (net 5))
 (segment (start 168.91 134.62) (end 168.91 140.72) (width 1) (layer B.Cu) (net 5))
 (segment (start 167.649999 128.010001) (end 167.649999 130.819999) (width 0.6) (layer B.Cu) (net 5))
 (segment (start 168.91 132.08) (end 170.18 130.81) (width 0.6) (layer B.Cu) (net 5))
 (segment (start 170.18 128.02) (end 169.16 127) (width 0.6) (layer B.Cu) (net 5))
 (segment (start 167.649999 130.819999) (end 168.91 132.08) (width 0.6) (layer B.Cu) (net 5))
 (segment (start 168.91 132.08) (end 168.91 134.62) (width 1) (layer B.Cu) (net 5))
 (segment (start 167.649999 141.999999) (end 168.150001 142.500001) (width 0.6) (layer F.Cu) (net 6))
 (segment (start 167.649999 139.690001) (end 167.649999 141.999999) (width 0.6) (layer F.Cu) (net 6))
 (segment (start 168.150001 142.500001) (end 168.91 143.26) (width 0.6) (layer F.Cu) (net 6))
 (segment (start 168.91 138.43) (end 167.649999 139.690001) (width 0.6) (layer F.Cu) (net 6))
 (segment (start 168.91 131.83) (end 168.91 138.43) (width 1) (layer F.Cu) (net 6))
 (segment (start 170.18 139.7) (end 170.18 142.24) (width 0.6) (layer F.Cu) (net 6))
 (segment (start 168.91 138.43) (end 170.18 139.7) (width 0.6) (layer F.Cu) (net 6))
 (segment (start 170.18 142.24) (end 168.91 143.51) (width 0.6) (layer F.Cu) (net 6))
 (segment (start 168.91 129.29) (end 168.91 131.83) (width 1) (layer F.Cu) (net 6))
 (segment (start 165.109999 130.819999) (end 166.37 132.08) (width 0.6) (layer F.Cu) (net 7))
 (segment (start 167.64 128.02) (end 166.62 127) (width 0.6) (layer F.Cu) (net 7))
 (segment (start 166.37 132.08) (end 167.64 130.81) (width 0.6) (layer F.Cu) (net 7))
 (segment (start 166.37 134.62) (end 166.37 140.72) (width 1) (layer F.Cu) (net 7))
 (segment (start 166.37 126.75) (end 165.109999 128.010001) (width 0.6) (layer F.Cu) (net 7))
 (segment (start 165.109999 128.010001) (end 165.109999 130.819999) (width 0.6) (layer F.Cu) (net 7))
 (segment (start 167.64 130.81) (end 167.64 128.02) (width 0.6) (layer F.Cu) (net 7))
 (segment (start 166.37 132.08) (end 166.37 134.62) (width 1) (layer F.Cu) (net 7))
 (segment (start 167.64 139.7) (end 167.64 142.24) (width 0.6) (layer B.Cu) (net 8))
 (segment (start 167.64 142.24) (end 166.37 143.51) (width 0.6) (layer B.Cu) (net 8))
 (segment (start 166.37 138.43) (end 165.109999 139.690001) (width 0.6) (layer B.Cu) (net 8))
 (segment (start 165.109999 141.999999) (end 165.610001 142.500001) (width 0.6) (layer B.Cu) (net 8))
 (segment (start 165.109999 139.690001) (end 165.109999 141.999999) (width 0.6) (layer B.Cu) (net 8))
 (segment (start 166.37 138.43) (end 167.64 139.7) (width 0.6) (layer B.Cu) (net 8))
 (segment (start 165.610001 142.500001) (end 166.37 143.26) (width 0.6) (layer B.Cu) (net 8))
 (segment (start 166.37 131.83) (end 166.37 138.43) (width 1) (layer B.Cu) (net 8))
 (segment (start 166.37 129.29) (end 166.37 131.83) (width 1) (layer B.Cu) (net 8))
 (segment (start 163.83 126.75) (end 162.569999 128.010001) (width 0.6) (layer B.Cu) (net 9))
 (segment (start 165.1 130.81) (end 165.1 128.02) (width 0.6) (layer B.Cu) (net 9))
 (segment (start 163.83 134.62) (end 163.83 140.72) (width 1) (layer B.Cu) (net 9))
 (segment (start 162.569999 128.010001) (end 162.569999 130.819999) (width 0.6) (layer B.Cu) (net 9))
 (segment (start 163.83 132.08) (end 165.1 130.81) (width 0.6) (layer B.Cu) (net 9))
 (segment (start 165.1 128.02) (end 164.08 127) (width 0.6) (layer B.Cu) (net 9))
 (segment (start 162.569999 130.819999) (end 163.83 132.08) (width 0.6) (layer B.Cu) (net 9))
 (segment (start 163.83 132.08) (end 163.83 134.62) (width 1) (layer B.Cu) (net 9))
 (segment (start 162.569999 141.999999) (end 163.070001 142.500001) (width 0.6) (layer F.Cu) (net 10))
 (segment (start 162.569999 139.690001) (end 162.569999 141.999999) (width 0.6) (layer F.Cu) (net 10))
 (segment (start 163.070001 142.500001) (end 163.83 143.26) (width 0.6) (layer F.Cu) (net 10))
 (segment (start 163.83 138.43) (end 162.569999 139.690001) (width 0.6) (layer F.Cu) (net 10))
 (segment (start 163.83 131.83) (end 163.83 138.43) (width 1) (layer F.Cu) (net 10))
 (segment (start 165.1 139.7) (end 165.1 142.24) (width 0.6) (layer F.Cu) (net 10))
 (segment (start 163.83 138.43) (end 165.1 139.7) (width 0.6) (layer F.Cu) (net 10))
 (segment (start 165.1 142.24) (end 163.83 143.51) (width 0.6) (layer F.Cu) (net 10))
 (segment (start 163.83 129.29) (end 163.83 131.83) (width 1) (layer F.Cu) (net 10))
 (segment (start 160.029999 130.819999) (end 161.29 132.08) (width 0.6) (layer F.Cu) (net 11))
 (segment (start 162.56 128.02) (end 161.54 127) (width 0.6) (layer F.Cu) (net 11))
 (segment (start 161.29 132.08) (end 162.56 130.81) (width 0.6) (layer F.Cu) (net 11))
 (segment (start 161.29 134.62) (end 161.29 140.72) (width 1) (layer F.Cu) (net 11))
 (segment (start 161.29 126.75) (end 160.029999 128.010001) (width 0.6) (layer F.Cu) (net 11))
 (segment (start 160.029999 128.010001) (end 160.029999 130.819999) (width 0.6) (layer F.Cu) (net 11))
 (segment (start 162.56 130.81) (end 162.56 128.02) (width 0.6) (layer F.Cu) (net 11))
 (segment (start 161.29 132.08) (end 161.29 134.62) (width 1) (layer F.Cu) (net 11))
 (segment (start 161.29 129.29) (end 161.29 131.83) (width 1) (layer B.Cu) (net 12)))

